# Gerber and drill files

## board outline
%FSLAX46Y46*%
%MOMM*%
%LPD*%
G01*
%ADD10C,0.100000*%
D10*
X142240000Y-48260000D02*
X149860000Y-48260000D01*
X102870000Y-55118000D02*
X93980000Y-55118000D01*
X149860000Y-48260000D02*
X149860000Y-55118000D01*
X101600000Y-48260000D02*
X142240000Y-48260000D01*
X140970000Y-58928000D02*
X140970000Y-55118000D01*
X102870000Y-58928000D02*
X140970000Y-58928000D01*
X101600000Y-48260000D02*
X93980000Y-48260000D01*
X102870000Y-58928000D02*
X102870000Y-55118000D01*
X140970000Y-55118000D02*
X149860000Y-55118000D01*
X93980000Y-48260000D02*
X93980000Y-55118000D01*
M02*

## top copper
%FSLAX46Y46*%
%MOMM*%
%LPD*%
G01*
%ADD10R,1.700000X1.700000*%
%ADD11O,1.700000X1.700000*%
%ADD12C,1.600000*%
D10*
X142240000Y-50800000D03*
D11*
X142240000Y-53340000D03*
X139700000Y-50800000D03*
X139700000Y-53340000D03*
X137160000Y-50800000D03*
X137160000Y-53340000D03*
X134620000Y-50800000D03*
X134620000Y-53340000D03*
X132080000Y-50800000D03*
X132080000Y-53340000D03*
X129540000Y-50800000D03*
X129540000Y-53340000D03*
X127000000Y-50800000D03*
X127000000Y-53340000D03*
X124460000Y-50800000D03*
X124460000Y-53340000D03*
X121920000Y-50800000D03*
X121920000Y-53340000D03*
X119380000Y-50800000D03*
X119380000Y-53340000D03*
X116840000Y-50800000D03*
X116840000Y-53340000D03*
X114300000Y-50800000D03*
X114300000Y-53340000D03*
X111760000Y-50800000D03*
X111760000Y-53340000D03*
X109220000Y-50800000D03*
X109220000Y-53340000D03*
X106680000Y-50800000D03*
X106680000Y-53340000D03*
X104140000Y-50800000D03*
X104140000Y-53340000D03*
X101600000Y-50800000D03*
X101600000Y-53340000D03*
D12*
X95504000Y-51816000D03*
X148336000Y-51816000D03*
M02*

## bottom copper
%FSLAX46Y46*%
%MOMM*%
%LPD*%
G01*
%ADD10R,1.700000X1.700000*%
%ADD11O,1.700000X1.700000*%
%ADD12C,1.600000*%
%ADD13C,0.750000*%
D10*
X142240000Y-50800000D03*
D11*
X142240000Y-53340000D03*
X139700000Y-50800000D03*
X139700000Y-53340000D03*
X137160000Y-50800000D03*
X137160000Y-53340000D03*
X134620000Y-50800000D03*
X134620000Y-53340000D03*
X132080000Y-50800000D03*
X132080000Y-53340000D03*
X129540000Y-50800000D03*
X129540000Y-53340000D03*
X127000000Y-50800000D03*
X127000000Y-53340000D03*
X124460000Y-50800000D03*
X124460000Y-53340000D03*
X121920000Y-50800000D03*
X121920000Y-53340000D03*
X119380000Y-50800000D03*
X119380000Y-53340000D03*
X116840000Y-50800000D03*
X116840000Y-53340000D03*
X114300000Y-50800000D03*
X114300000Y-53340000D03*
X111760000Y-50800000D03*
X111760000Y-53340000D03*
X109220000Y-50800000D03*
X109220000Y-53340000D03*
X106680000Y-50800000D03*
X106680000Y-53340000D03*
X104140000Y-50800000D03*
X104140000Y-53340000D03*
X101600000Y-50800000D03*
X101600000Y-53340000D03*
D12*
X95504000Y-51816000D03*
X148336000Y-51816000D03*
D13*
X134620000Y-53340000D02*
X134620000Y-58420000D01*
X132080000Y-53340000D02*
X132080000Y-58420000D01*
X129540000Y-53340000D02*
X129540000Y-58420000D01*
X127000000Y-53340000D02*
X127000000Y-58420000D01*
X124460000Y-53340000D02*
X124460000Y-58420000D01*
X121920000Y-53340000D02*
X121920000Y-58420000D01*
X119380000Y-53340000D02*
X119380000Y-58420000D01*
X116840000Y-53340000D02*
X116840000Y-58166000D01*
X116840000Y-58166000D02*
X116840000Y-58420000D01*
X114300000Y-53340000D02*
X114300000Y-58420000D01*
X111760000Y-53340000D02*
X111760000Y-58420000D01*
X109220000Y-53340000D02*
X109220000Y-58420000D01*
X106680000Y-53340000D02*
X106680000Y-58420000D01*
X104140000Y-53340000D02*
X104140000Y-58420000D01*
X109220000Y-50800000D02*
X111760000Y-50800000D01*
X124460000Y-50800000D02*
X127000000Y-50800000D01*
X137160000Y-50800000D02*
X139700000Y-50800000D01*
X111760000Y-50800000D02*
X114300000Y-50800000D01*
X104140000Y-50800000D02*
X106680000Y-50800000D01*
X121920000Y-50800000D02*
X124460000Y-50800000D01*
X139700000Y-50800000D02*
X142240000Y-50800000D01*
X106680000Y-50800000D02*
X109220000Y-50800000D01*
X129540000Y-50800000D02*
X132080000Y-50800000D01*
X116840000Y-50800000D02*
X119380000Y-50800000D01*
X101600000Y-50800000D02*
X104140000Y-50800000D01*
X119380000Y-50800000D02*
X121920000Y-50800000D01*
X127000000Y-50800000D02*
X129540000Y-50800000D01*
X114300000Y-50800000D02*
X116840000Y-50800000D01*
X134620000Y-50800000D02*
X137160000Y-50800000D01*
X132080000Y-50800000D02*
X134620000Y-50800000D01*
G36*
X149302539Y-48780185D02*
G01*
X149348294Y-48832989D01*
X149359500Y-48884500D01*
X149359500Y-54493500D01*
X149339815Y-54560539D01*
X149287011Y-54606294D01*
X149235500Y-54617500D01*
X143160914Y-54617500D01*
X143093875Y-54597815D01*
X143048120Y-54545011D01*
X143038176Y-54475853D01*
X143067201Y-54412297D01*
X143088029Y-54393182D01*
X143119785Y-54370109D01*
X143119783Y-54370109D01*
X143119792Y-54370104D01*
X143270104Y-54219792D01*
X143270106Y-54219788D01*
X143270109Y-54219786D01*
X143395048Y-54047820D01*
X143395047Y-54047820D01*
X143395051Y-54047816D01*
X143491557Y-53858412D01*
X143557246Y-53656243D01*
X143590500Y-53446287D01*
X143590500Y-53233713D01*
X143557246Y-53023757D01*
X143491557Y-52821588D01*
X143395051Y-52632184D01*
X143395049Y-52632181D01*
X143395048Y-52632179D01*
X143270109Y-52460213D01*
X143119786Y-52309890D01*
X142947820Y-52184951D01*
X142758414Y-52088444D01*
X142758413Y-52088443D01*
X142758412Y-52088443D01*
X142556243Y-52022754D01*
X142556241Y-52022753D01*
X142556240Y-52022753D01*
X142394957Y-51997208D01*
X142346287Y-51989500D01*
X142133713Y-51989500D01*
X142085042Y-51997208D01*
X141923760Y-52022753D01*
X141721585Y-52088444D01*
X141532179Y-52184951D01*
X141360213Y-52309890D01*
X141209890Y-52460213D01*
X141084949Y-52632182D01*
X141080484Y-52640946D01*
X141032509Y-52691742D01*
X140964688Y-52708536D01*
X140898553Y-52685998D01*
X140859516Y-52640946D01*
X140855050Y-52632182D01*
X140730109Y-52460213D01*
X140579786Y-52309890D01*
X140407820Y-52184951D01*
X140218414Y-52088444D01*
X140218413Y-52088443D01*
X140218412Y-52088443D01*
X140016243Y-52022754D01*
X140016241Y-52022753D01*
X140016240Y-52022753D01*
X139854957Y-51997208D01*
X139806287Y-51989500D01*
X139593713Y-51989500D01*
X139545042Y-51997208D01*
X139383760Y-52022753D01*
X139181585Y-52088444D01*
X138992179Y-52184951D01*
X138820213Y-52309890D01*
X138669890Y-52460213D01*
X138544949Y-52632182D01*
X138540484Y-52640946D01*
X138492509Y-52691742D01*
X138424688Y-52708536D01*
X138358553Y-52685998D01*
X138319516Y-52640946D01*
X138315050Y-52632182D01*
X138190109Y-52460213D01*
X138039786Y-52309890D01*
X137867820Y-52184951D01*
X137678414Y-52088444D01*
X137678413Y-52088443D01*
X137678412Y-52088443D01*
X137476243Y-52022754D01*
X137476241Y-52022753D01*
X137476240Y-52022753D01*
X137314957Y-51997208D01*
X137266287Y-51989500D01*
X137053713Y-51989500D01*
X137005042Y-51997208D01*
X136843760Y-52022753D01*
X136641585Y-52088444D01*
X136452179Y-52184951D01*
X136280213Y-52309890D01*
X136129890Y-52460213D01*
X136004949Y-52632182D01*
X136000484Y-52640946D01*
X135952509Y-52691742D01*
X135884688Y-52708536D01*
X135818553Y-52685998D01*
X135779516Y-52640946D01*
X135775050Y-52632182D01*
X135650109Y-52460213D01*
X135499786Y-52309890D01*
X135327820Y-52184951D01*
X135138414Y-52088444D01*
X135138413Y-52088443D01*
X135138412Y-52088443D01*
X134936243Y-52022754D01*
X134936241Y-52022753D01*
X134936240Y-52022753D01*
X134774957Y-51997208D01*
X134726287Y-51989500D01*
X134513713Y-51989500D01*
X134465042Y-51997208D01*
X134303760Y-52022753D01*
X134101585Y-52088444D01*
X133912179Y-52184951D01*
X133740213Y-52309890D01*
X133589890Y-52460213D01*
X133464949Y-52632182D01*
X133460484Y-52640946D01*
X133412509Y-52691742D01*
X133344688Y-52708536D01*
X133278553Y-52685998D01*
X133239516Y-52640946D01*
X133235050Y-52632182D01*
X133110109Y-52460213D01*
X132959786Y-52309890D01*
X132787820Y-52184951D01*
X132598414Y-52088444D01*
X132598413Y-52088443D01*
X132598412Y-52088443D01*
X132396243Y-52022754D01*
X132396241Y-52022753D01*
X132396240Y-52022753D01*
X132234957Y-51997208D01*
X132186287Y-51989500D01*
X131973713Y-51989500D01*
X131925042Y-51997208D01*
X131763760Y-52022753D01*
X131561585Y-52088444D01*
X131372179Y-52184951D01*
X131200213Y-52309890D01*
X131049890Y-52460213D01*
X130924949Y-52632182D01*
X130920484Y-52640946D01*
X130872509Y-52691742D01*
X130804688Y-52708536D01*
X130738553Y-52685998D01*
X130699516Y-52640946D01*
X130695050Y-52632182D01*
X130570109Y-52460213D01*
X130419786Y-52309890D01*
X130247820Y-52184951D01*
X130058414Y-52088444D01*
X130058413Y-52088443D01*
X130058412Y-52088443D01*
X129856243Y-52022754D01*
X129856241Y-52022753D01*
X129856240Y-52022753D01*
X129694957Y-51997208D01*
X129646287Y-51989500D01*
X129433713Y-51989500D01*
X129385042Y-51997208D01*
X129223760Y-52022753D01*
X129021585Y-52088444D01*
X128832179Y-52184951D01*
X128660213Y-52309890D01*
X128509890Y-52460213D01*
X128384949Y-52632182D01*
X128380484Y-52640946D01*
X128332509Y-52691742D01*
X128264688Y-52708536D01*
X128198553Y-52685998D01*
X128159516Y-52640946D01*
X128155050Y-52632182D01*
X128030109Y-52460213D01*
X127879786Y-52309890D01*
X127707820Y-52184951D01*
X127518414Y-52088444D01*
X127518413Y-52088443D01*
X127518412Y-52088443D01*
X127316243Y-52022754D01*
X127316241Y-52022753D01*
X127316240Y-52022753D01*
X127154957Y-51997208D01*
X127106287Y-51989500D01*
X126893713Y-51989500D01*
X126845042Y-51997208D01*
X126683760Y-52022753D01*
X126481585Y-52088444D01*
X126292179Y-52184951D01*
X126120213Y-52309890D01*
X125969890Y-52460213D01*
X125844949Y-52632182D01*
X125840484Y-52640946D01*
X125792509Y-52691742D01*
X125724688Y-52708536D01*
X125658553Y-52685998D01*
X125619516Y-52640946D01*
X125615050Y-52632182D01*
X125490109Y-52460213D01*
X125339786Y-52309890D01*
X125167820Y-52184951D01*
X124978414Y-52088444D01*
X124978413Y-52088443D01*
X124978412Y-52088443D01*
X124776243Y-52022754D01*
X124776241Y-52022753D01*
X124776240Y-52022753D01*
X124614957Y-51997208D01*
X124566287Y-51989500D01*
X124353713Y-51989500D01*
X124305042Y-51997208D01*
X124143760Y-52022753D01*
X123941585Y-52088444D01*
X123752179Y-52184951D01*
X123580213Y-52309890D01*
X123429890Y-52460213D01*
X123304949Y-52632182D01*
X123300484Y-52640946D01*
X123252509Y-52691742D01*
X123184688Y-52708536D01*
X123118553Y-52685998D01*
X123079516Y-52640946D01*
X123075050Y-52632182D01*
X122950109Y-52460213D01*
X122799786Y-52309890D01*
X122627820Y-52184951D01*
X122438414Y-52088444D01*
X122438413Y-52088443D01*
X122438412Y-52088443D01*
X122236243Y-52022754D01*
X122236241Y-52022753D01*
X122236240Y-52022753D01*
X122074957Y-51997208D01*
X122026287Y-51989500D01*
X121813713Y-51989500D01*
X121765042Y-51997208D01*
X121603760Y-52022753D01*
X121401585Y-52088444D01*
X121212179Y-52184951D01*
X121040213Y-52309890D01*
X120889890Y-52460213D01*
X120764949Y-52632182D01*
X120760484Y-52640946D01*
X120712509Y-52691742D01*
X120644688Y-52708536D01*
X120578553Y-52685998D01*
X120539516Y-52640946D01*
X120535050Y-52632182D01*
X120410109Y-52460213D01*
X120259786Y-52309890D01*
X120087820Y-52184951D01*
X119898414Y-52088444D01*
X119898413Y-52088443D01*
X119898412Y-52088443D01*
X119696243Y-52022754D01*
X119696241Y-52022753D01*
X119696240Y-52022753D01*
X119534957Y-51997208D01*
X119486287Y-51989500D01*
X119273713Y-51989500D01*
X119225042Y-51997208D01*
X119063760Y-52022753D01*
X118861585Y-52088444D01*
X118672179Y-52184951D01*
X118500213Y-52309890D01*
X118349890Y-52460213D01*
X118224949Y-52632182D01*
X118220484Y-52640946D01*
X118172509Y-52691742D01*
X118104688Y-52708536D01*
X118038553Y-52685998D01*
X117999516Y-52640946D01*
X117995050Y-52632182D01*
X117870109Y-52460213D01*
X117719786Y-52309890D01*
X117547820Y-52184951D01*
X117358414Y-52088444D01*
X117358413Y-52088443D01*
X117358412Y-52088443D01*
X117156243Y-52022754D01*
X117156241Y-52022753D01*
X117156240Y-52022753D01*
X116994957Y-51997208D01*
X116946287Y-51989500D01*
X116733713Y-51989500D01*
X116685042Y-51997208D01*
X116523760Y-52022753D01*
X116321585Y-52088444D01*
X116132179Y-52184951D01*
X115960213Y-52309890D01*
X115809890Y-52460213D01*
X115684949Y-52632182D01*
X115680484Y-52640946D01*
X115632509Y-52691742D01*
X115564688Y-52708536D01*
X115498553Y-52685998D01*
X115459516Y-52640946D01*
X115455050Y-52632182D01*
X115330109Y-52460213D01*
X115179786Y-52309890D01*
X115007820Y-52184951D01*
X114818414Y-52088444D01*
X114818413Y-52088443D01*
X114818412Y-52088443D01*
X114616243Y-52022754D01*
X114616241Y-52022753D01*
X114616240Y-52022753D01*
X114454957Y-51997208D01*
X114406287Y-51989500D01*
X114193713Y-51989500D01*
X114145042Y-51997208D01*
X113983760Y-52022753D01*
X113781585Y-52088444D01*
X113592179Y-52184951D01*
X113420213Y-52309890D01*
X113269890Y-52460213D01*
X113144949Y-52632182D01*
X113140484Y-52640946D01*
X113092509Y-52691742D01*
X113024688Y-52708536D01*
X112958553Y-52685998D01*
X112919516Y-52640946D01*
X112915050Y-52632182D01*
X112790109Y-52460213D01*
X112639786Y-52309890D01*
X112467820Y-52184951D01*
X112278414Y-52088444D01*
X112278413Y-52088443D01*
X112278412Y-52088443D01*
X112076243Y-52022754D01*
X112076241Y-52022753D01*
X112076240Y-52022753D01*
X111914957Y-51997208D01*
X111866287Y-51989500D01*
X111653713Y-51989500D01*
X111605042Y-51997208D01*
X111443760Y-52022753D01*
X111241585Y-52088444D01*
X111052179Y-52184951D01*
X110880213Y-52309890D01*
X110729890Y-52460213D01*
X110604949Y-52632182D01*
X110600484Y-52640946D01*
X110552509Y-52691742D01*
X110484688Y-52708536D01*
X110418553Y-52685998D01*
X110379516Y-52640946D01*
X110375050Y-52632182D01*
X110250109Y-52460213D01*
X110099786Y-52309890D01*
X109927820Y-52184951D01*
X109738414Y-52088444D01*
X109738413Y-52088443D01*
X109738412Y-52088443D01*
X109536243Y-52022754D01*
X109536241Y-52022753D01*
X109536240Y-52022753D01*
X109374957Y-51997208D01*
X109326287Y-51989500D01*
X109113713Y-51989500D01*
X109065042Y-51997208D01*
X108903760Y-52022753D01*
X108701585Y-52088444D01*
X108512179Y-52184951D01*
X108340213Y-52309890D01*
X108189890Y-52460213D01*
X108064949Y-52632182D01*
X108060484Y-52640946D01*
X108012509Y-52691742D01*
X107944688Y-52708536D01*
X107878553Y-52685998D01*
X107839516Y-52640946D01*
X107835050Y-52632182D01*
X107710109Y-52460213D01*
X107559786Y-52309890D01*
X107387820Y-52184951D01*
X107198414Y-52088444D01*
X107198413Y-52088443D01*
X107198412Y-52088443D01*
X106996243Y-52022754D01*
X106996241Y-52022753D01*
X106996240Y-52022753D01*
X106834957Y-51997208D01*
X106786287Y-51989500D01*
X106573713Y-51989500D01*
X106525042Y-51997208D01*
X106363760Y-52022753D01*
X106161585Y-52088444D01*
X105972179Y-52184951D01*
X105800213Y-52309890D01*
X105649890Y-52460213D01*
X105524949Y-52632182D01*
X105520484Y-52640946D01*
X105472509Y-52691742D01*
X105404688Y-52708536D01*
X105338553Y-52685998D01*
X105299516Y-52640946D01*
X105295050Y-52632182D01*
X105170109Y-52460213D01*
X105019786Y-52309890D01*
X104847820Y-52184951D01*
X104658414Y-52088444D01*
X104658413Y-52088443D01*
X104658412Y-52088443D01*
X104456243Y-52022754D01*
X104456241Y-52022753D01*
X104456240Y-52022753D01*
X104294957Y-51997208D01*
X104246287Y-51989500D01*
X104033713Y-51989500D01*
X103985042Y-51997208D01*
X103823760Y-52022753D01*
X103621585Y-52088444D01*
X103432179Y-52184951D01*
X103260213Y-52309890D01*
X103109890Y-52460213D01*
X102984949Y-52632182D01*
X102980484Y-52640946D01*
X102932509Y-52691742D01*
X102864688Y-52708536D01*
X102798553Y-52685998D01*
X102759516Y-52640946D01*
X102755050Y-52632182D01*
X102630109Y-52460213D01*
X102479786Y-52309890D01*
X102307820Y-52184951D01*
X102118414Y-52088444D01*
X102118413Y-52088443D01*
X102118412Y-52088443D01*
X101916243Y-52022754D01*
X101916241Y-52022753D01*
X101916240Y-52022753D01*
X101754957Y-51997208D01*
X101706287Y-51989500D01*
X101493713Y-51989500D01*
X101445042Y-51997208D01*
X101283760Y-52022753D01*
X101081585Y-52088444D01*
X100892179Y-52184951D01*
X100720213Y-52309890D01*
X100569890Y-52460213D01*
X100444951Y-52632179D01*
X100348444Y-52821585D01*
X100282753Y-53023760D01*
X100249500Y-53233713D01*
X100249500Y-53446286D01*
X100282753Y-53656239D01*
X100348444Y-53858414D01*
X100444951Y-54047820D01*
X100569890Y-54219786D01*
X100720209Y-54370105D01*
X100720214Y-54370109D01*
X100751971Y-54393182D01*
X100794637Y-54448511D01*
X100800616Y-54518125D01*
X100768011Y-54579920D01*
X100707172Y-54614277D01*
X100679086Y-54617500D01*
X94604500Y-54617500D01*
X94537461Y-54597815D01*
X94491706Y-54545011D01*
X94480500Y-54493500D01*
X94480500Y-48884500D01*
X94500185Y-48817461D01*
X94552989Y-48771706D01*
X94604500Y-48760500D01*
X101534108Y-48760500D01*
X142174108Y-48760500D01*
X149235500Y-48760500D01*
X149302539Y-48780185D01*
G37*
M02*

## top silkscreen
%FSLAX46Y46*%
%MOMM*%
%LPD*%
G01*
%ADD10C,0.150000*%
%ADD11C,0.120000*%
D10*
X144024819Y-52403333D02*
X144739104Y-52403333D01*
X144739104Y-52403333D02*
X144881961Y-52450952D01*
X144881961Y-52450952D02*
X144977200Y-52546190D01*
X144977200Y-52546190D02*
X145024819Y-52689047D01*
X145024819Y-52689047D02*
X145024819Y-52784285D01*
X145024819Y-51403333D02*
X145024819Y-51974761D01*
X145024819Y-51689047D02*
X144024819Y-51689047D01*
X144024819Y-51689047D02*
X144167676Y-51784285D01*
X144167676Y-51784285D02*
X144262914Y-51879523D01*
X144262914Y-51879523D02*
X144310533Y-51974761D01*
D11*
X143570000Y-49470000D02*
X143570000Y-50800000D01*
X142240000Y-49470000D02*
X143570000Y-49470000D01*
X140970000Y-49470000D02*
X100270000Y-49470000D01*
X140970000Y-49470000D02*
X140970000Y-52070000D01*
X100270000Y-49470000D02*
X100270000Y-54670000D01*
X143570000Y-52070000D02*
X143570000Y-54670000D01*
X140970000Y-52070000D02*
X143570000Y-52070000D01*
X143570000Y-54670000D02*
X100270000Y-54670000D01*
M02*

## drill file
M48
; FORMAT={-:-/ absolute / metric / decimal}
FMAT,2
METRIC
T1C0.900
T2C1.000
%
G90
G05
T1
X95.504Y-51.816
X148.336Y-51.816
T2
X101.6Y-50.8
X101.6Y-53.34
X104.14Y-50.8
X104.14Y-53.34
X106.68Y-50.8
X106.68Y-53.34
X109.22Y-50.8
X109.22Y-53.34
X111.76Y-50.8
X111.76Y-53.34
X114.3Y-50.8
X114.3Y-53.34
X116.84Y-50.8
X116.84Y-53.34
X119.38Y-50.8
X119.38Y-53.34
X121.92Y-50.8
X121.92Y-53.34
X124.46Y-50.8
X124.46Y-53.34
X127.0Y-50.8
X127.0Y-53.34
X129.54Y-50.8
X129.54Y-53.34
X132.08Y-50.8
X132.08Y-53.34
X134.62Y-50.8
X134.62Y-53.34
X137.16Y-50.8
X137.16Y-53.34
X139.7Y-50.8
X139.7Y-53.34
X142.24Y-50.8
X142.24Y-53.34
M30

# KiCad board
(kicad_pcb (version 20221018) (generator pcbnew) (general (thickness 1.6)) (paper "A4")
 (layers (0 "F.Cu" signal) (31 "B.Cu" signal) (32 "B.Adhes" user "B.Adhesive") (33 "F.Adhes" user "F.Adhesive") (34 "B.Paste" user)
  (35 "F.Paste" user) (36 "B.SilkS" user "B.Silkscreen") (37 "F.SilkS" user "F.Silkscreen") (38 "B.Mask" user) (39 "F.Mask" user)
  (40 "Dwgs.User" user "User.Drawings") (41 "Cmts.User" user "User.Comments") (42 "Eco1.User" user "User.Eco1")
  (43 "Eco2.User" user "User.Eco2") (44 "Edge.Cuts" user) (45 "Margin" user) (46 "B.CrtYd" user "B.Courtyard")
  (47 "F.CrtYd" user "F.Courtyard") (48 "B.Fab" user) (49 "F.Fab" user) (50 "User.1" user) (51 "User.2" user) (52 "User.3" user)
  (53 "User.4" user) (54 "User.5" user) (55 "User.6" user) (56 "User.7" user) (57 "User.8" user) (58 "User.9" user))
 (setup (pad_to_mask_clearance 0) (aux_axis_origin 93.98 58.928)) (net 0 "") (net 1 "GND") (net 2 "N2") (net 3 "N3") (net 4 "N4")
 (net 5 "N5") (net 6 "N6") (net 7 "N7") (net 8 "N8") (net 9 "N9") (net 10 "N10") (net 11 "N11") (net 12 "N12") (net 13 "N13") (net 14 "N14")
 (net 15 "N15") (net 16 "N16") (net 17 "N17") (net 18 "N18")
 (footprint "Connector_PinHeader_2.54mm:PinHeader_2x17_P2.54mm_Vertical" (layer "F.Cu") (at 142.24 50.8 -90)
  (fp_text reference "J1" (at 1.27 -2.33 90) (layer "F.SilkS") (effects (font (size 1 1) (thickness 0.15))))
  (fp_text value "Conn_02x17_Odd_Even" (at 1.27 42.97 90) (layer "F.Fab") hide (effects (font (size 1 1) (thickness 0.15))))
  (fp_line (start -1.33 -1.33) (end 0 -1.33) (stroke (width 0.12) (type solid)) (layer "F.SilkS"))
  (fp_line (start -1.33 0) (end -1.33 -1.33) (stroke (width 0.12) (type solid)) (layer "F.SilkS"))
  (fp_line (start -1.33 1.27) (end -1.33 41.97) (stroke (width 0.12) (type solid)) (layer "F.SilkS"))
  (fp_line (start -1.33 1.27) (end 1.27 1.27) (stroke (width 0.12) (type solid)) (layer "F.SilkS"))
  (fp_line (start -1.33 41.97) (end 3.87 41.97) (stroke (width 0.12) (type solid)) (layer "F.SilkS"))
  (fp_line (start 1.27 -1.33) (end 3.87 -1.33) (stroke (width 0.12) (type solid)) (layer "F.SilkS"))
  (fp_line (start 1.27 1.27) (end 1.27 -1.33) (stroke (width 0.12) (type solid)) (layer "F.SilkS"))
  (fp_line (start 3.87 -1.33) (end 3.87 41.97) (stroke (width 0.12) (type solid)) (layer "F.SilkS"))
  (pad "1" thru_hole rect (at 0 0 270) (size 1.7 1.7) (drill 1) (layers "*.Cu" "*.Mask") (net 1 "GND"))
  (pad "2" thru_hole oval (at 2.54 0 270) (size 1.7 1.7) (drill 1) (layers "*.Cu" "*.Mask") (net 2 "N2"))
  (pad "3" thru_hole oval (at 0 2.54 270) (size 1.7 1.7) (drill 1) (layers "*.Cu" "*.Mask") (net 1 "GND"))
  (pad "4" thru_hole oval (at 2.54 2.54 270) (size 1.7 1.7) (drill 1) (layers "*.Cu" "*.Mask") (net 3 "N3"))
  (pad "5" thru_hole oval (at 0 5.08 270) (size 1.7 1.7) (drill 1) (layers "*.Cu" "*.Mask") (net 1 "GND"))
  (pad "6" thru_hole oval (at 2.54 5.08 270) (size 1.7 1.7) (drill 1) (layers "*.Cu" "*.Mask") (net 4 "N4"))
  (pad "7" thru_hole oval (at 0 7.62 270) (size 1.7 1.7) (drill 1) (layers "*.Cu" "*.Mask") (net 1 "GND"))
  (pad "8" thru_hole oval (at 2.54 7.62 270) (size 1.7 1.7) (drill 1) (layers "*.Cu" "*.Mask") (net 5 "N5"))
  (pad "9" thru_hole oval (at 0 10.16 270) (size 1.7 1.7) (drill 1) (layers "*.Cu" "*.Mask") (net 1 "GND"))
  (pad "10" thru_hole oval (at 2.54 10.16 270) (size 1.7 1.7) (drill 1) (layers "*.Cu" "*.Mask") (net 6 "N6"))
  (pad "11" thru_hole oval (at 0 12.7 270) (size 1.7 1.7) (drill 1) (layers "*.Cu" "*.Mask") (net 1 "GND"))
  (pad "12" thru_hole oval (at 2.54 12.7 270) (size 1.7 1.7) (drill 1) (layers "*.Cu" "*.Mask") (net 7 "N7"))
  (pad "13" thru_hole oval (at 0 15.24 270) (size 1.7 1.7) (drill 1) (layers "*.Cu" "*.Mask") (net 1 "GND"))
  (pad "14" thru_hole oval (at 2.54 15.24 270) (size 1.7 1.7) (drill 1) (layers "*.Cu" "*.Mask") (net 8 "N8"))
  (pad "15" thru_hole oval (at 0 17.78 270) (size 1.7 1.7) (drill 1) (layers "*.Cu" "*.Mask") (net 1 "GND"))
  (pad "16" thru_hole oval (at 2.54 17.78 270) (size 1.7 1.7) (drill 1) (layers "*.Cu" "*.Mask") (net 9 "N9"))
  (pad "17" thru_hole oval (at 0 20.32 270) (size 1.7 1.7) (drill 1) (layers "*.Cu" "*.Mask") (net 1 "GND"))
  (pad "18" thru_hole oval (at 2.54 20.32 270) (size 1.7 1.7) (drill 1) (layers "*.Cu" "*.Mask") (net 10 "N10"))
  (pad "19" thru_hole oval (at 0 22.86 270) (size 1.7 1.7) (drill 1) (layers "*.Cu" "*.Mask") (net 1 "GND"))
  (pad "20" thru_hole oval (at 2.54 22.86 270) (size 1.7 1.7) (drill 1) (layers "*.Cu" "*.Mask") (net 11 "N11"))
  (pad "21" thru_hole oval (at 0 25.4 270) (size 1.7 1.7) (drill 1) (layers "*.Cu" "*.Mask") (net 1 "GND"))
  (pad "22" thru_hole oval (at 2.54 25.4 270) (size 1.7 1.7) (drill 1) (layers "*.Cu" "*.Mask") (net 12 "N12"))
  (pad "23" thru_hole oval (at 0 27.94 270) (size 1.7 1.7) (drill 1) (layers "*.Cu" "*.Mask") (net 1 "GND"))
  (pad "24" thru_hole oval (at 2.54 27.94 270) (size 1.7 1.7) (drill 1) (layers "*.Cu" "*.Mask") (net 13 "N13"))
  (pad "25" thru_hole oval (at 0 30.48 270) (size 1.7 1.7) (drill 1) (layers "*.Cu" "*.Mask") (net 1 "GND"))
  (pad "26" thru_hole oval (at 2.54 30.48 270) (size 1.7 1.7) (drill 1) (layers "*.Cu" "*.Mask") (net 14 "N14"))
  (pad "27" thru_hole oval (at 0 33.02 270) (size 1.7 1.7) (drill 1) (layers "*.Cu" "*.Mask") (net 1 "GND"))
  (pad "28" thru_hole oval (at 2.54 33.02 270) (size 1.7 1.7) (drill 1) (layers "*.Cu" "*.Mask") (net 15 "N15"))
  (pad "29" thru_hole oval (at 0 35.56 270) (size 1.7 1.7) (drill 1) (layers "*.Cu" "*.Mask") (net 1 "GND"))
  (pad "30" thru_hole oval (at 2.54 35.56 270) (size 1.7 1.7) (drill 1) (layers "*.Cu" "*.Mask") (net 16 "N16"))
  (pad "31" thru_hole oval (at 0 38.1 270) (size 1.7 1.7) (drill 1) (layers "*.Cu" "*.Mask") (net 1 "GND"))
  (pad "32" thru_hole oval (at 2.54 38.1 270) (size 1.7 1.7) (drill 1) (layers "*.Cu" "*.Mask") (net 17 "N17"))
  (pad "33" thru_hole oval (at 0 40.64 270) (size 1.7 1.7) (drill 1) (layers "*.Cu" "*.Mask") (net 1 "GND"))
  (pad "34" thru_hole oval (at 2.54 40.64 270) (size 1.7 1.7) (drill 1) (layers "*.Cu" "*.Mask") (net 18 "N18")))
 (gr_line (start 142.24 48.26) (end 149.86 48.26) (stroke (width 0.1) (type default)) (layer "Edge.Cuts"))
 (gr_line (start 102.87 55.118) (end 93.98 55.118) (stroke (width 0.1) (type default)) (layer "Edge.Cuts"))
 (gr_line (start 149.86 48.26) (end 149.86 55.118) (stroke (width 0.1) (type default)) (layer "Edge.Cuts"))
 (gr_line (start 101.6 48.26) (end 142.24 48.26) (stroke (width 0.1) (type default)) (layer "Edge.Cuts"))
 (gr_line (start 140.97 58.928) (end 140.97 55.118) (stroke (width 0.1) (type default)) (layer "Edge.Cuts"))
 (gr_line (start 102.87 58.928) (end 140.97 58.928) (stroke (width 0.1) (type default)) (layer "Edge.Cuts"))
 (gr_line (start 101.6 48.26) (end 93.98 48.26) (stroke (width 0.1) (type default)) (layer "Edge.Cuts"))
 (gr_line (start 102.87 58.928) (end 102.87 55.118) (stroke (width 0.1) (type default)) (layer "Edge.Cuts"))
 (gr_line (start 140.97 55.118) (end 149.86 55.118) (stroke (width 0.1) (type default)) (layer "Edge.Cuts"))
 (gr_line (start 93.98 48.26) (end 93.98 55.118) (stroke (width 0.1) (type default)) (layer "Edge.Cuts"))
 (segment (start 134.62 53.34) (end 134.62 58.42) (width 0.75) (layer "B.Cu") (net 5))
 (segment (start 132.08 53.34) (end 132.08 58.42) (width 0.75) (layer "B.Cu") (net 6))
 (segment (start 129.54 53.34) (end 129.54 58.42) (width 0.75) (layer "B.Cu") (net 7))
 (segment (start 127 53.34) (end 127 58.42) (width 0.75) (layer "B.Cu") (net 8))
 (segment (start 124.46 53.34) (end 124.46 58.42) (width 0.75) (layer "B.Cu") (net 9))
 (segment (start 121.92 53.34) (end 121.92 58.42) (width 0.75) (layer "B.Cu") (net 10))
 (segment (start 119.38 53.34) (end 119.38 58.42) (width 0.75) (layer "B.Cu") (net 11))
 (segment (start 116.84 53.34) (end 116.84 58.166) (width 0.75) (layer "B.Cu") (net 12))
 (segment (start 116.84 58.166) (end 116.84 58.42) (width 0.75) (layer "B.Cu") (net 12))
 (segment (start 114.3 53.34) (end 114.3 58.42) (width 0.75) (layer "B.Cu") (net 13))
 (segment (start 111.76 53.34) (end 111.76 58.42) (width 0.75) (layer "B.Cu") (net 14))
 (segment (start 109.22 53.34) (end 109.22 58.42) (width 0.75) (layer "B.Cu") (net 15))
 (segment (start 106.68 53.34) (end 106.68 58.42) (width 0.75) (layer "B.Cu") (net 16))
 (segment (start 104.14 53.34) (end 104.14 58.42) (width 0.75) (layer "B.Cu") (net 17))
 (via (at 95.504 51.816) (size 1.6) (drill 0.9) (layers "F.Cu" "B.Cu") (free) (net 1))
 (via (at 148.336 51.816) (size 1.6) (drill 0.9) (layers "F.Cu" "B.Cu") (free) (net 1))
 (segment (start 109.22 50.8) (end 111.76 50.8) (width 0.75) (layer "B.Cu") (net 1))
 (segment (start 124.46 50.8) (end 127 50.8) (width 0.75) (layer "B.Cu") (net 1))
 (segment (start 137.16 50.8) (end 139.7 50.8) (width 0.75) (layer "B.Cu") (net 1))
 (segment (start 111.76 50.8) (end 114.3 50.8) (width 0.75) (layer "B.Cu") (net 1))
 (segment (start 104.14 50.8) (end 106.68 50.8) (width 0.75) (layer "B.Cu") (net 1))
 (segment (start 121.92 50.8) (end 124.46 50.8) (width 0.75) (layer "B.Cu") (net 1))
 (segment (start 139.7 50.8) (end 142.24 50.8) (width 0.75) (layer "B.Cu") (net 1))
 (segment (start 106.68 50.8) (end 109.22 50.8) (width 0.75) (layer "B.Cu") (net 1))
 (segment (start 129.54 50.8) (end 132.08 50.8) (width 0.75) (layer "B.Cu") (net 1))
 (segment (start 116.84 50.8) (end 119.38 50.8) (width 0.75) (layer "B.Cu") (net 1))
 (segment (start 101.6 50.8) (end 104.14 50.8) (width 0.75) (layer "B.Cu") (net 1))
 (segment (start 119.38 50.8) (end 121.92 50.8) (width 0.75) (layer "B.Cu") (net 1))
 (segment (start 127 50.8) (end 129.54 50.8) (width 0.75) (layer "B.Cu") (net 1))
 (segment (start 114.3 50.8) (end 116.84 50.8) (width 0.75) (layer "B.Cu") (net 1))
 (segment (start 134.62 50.8) (end 137.16 50.8) (width 0.75) (layer "B.Cu") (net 1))
 (segment (start 132.08 50.8) (end 134.62 50.8) (width 0.75) (layer "B.Cu") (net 1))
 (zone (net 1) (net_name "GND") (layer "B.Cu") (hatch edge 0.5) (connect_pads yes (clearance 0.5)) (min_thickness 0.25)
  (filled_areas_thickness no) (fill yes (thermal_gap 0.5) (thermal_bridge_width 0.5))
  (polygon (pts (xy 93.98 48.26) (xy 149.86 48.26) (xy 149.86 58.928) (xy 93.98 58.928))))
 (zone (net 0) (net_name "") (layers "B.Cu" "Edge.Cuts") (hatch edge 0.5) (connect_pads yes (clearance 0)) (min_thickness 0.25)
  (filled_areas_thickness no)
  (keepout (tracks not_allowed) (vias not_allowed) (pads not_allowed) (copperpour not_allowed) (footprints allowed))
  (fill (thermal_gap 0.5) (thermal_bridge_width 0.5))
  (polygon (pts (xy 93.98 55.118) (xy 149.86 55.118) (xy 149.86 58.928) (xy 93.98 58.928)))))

